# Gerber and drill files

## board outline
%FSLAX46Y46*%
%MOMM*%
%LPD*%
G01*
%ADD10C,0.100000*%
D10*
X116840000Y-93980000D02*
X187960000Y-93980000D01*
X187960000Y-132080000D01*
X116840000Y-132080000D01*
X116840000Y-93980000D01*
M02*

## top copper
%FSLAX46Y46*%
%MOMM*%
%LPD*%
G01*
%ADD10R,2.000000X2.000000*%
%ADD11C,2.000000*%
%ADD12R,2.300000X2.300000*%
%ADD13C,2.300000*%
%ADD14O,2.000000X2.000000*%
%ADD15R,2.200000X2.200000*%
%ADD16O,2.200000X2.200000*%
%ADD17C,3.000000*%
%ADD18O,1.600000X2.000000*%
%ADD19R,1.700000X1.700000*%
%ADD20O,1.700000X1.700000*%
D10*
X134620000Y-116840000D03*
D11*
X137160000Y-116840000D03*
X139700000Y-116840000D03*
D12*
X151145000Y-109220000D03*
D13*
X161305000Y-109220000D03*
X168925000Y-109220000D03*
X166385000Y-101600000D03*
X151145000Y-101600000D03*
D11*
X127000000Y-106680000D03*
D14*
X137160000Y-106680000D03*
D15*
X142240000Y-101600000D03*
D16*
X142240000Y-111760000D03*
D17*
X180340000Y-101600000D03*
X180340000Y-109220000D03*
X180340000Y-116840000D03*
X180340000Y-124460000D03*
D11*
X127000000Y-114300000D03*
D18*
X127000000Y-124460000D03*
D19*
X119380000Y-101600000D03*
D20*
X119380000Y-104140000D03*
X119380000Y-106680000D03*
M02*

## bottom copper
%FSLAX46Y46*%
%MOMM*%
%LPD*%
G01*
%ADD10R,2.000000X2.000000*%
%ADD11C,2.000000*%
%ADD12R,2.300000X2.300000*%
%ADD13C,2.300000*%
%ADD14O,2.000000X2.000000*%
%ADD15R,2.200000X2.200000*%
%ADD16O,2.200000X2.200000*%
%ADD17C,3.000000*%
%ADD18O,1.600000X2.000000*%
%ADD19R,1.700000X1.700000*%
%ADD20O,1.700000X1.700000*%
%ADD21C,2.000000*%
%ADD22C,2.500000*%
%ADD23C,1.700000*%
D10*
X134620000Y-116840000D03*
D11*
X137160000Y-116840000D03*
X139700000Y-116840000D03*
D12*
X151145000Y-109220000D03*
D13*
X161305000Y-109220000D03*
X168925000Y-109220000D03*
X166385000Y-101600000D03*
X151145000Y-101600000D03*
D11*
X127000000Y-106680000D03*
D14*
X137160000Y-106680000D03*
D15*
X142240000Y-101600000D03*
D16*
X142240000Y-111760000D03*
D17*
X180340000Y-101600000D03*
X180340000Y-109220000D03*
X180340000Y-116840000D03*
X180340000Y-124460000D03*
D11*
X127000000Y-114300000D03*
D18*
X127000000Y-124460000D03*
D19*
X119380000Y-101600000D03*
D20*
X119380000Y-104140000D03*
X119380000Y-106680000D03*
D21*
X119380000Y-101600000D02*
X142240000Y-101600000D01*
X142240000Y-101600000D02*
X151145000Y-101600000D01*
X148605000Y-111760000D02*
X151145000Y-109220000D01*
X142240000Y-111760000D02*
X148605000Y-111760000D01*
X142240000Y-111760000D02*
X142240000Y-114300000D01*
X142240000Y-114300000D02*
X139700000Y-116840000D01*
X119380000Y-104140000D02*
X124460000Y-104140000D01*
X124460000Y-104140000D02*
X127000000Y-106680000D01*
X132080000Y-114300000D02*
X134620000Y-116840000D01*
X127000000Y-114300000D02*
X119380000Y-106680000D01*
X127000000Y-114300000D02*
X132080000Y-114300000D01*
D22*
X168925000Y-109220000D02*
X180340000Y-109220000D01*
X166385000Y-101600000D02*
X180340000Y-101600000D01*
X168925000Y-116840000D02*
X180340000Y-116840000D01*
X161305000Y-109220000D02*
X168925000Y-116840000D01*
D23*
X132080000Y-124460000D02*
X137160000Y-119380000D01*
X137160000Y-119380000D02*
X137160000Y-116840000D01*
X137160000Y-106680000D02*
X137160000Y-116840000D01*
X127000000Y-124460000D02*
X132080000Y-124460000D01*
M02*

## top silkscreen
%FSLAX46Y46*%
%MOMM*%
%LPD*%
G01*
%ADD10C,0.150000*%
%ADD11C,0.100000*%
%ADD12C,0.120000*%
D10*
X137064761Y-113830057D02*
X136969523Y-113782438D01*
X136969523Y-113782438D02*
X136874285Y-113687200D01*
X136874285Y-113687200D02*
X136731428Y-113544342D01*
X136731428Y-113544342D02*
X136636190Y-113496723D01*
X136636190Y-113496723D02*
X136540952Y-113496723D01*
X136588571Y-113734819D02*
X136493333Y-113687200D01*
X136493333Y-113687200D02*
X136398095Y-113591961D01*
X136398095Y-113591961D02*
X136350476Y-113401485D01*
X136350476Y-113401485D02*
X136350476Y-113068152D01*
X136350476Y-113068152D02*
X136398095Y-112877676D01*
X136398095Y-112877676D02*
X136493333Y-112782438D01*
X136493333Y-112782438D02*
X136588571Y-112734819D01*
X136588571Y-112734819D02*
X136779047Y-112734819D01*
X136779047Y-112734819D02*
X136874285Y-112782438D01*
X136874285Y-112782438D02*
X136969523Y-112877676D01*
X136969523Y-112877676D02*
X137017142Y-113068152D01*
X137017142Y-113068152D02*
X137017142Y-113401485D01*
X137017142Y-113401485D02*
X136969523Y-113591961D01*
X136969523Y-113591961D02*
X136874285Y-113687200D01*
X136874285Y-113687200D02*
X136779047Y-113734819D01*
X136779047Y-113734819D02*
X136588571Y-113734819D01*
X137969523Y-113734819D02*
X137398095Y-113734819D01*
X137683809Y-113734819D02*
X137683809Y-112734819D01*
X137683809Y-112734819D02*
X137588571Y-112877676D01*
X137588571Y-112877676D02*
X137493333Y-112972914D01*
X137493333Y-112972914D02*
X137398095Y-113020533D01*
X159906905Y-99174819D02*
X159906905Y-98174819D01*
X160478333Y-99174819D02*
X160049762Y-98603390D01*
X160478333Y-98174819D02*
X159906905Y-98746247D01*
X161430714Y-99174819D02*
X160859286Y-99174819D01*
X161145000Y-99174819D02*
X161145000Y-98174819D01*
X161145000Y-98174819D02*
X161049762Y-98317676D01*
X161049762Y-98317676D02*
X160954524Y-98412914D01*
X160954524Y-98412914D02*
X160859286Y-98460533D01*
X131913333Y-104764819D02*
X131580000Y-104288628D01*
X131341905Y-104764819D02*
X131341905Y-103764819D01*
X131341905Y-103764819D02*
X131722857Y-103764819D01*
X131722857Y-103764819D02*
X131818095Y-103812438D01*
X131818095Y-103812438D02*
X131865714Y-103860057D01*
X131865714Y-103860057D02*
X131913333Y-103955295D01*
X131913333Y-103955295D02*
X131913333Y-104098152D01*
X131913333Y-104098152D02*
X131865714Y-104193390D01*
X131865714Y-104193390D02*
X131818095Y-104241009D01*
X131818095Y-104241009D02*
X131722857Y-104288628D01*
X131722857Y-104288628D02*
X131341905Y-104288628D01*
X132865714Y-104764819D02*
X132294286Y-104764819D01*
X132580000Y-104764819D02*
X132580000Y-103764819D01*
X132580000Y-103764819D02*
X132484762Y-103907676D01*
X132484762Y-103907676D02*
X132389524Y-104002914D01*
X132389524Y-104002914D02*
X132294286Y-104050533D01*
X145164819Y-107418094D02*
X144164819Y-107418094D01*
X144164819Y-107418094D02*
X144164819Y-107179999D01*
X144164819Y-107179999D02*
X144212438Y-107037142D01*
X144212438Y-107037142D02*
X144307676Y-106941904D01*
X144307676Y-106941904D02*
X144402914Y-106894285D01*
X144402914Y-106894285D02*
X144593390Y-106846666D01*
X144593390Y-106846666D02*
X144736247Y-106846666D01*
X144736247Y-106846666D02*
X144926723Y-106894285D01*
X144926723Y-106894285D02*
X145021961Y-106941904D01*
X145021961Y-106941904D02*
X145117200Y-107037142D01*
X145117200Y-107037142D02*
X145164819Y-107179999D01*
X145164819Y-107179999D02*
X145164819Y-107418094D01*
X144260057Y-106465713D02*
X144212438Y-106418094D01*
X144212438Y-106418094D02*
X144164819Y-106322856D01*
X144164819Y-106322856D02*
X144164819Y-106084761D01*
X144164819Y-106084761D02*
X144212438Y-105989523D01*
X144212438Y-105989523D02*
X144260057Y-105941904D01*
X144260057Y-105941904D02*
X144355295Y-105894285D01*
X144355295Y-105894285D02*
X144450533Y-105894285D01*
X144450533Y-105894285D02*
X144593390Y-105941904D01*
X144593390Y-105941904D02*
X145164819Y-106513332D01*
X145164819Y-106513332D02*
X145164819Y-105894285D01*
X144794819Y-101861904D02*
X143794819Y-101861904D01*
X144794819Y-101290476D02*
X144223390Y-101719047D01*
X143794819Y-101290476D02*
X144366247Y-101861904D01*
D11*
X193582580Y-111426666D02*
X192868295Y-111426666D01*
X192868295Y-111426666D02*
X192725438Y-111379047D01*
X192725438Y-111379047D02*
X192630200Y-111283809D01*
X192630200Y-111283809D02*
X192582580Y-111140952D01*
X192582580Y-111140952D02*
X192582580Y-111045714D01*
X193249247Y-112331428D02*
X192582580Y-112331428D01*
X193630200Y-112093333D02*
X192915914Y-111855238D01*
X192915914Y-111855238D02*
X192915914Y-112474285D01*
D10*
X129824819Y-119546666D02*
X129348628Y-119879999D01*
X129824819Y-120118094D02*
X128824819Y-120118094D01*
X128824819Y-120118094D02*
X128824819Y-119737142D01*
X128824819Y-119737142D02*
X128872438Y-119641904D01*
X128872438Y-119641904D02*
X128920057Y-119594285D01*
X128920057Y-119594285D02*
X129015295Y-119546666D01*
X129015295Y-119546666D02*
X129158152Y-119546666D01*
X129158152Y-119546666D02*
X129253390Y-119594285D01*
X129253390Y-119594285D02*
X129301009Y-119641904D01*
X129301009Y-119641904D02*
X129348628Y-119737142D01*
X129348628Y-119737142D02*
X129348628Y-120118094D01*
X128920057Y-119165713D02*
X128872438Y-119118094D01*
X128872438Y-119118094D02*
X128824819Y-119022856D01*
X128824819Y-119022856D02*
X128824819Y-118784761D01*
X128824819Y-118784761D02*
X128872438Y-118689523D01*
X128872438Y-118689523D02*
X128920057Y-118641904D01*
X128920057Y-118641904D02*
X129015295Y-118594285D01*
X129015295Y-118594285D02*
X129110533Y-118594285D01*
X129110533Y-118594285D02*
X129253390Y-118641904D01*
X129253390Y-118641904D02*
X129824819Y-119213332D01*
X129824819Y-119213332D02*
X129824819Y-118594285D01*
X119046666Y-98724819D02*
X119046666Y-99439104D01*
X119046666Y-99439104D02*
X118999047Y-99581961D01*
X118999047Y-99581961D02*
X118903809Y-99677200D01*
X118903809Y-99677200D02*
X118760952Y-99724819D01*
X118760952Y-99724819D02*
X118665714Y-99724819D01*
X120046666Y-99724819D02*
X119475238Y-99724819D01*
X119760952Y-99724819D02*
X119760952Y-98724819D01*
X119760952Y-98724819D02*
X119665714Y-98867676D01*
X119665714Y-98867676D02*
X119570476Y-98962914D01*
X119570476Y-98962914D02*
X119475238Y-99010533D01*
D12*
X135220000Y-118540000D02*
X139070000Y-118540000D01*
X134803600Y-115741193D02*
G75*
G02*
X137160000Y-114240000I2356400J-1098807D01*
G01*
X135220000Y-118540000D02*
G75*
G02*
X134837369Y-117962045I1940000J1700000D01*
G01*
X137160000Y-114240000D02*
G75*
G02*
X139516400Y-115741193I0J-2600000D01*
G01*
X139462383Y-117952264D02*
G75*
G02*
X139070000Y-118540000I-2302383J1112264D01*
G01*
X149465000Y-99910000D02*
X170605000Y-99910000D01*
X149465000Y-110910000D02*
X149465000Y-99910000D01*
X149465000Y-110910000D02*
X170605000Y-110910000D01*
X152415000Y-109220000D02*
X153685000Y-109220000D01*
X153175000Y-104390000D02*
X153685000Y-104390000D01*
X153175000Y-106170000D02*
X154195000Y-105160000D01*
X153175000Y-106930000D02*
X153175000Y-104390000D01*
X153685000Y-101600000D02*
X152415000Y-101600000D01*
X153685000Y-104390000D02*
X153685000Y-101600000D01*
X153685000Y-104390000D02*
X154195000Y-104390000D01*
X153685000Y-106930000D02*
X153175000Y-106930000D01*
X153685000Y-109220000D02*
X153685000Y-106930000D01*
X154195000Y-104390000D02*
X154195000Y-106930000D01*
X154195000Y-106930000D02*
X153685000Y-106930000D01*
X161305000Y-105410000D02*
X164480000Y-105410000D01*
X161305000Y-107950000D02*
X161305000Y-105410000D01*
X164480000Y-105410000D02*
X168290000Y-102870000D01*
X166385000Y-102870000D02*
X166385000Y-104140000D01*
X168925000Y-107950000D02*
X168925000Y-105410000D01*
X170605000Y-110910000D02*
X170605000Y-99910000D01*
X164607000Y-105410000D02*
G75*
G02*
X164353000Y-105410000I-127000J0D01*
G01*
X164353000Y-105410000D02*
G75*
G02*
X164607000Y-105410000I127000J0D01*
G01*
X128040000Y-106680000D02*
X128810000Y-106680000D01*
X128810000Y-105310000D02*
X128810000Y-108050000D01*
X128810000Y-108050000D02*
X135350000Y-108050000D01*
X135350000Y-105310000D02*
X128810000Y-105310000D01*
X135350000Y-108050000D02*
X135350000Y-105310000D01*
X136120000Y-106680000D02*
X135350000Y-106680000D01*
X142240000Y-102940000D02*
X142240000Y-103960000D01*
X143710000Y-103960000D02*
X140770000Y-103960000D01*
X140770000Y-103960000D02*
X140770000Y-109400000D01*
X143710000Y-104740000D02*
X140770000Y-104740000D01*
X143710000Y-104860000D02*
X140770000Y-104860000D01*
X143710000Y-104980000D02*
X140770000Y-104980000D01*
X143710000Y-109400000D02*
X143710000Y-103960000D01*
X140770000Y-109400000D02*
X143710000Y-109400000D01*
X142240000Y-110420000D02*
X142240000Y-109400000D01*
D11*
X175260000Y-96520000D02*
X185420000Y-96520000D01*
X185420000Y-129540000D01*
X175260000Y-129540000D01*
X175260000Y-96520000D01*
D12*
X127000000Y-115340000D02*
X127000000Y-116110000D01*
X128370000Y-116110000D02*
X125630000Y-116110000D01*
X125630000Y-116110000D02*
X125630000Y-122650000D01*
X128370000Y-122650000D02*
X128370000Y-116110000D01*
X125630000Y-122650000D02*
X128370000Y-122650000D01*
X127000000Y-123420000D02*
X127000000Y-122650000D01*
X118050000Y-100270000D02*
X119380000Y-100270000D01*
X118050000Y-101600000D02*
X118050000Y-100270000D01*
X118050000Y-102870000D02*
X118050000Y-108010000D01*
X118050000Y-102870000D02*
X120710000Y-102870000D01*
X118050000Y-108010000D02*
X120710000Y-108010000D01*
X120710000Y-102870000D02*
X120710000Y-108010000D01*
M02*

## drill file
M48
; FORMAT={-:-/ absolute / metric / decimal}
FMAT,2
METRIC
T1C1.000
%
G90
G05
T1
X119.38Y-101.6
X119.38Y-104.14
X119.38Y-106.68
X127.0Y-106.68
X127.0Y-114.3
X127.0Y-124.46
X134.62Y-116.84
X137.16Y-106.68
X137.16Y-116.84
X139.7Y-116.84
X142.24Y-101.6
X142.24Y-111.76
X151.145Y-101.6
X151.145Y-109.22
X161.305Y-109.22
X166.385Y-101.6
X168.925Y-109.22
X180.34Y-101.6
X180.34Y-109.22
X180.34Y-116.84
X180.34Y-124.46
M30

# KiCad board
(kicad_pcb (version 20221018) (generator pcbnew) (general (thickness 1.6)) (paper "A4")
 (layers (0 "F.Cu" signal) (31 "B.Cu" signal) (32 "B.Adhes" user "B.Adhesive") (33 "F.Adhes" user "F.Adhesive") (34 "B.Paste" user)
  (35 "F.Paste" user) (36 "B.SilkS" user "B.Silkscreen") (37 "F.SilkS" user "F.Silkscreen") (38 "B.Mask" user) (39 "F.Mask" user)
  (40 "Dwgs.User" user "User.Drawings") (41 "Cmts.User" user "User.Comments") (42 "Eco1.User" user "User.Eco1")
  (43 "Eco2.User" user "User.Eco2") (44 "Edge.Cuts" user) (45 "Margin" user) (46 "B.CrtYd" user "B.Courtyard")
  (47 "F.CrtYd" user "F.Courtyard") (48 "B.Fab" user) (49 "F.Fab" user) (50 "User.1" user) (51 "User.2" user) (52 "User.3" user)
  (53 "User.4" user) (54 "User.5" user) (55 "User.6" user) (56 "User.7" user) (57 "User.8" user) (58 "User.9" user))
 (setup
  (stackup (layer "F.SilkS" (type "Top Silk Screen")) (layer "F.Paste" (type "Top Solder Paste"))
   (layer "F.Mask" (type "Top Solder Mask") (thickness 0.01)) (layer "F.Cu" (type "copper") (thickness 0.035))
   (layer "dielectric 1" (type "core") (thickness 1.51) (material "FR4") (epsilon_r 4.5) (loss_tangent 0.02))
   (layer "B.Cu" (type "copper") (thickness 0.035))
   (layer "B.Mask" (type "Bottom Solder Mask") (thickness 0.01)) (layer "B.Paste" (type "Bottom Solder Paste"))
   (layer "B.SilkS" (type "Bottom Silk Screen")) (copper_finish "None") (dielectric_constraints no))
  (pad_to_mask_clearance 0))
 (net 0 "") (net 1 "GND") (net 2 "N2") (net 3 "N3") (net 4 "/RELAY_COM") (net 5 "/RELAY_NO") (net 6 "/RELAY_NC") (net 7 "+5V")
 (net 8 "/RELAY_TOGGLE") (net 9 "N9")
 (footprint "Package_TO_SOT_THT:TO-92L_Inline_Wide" (layer "F.Cu") (at 134.62 116.84)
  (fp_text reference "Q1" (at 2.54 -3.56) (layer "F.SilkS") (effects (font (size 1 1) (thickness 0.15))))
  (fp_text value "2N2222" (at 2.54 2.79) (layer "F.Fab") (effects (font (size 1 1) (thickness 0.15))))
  (fp_line (start 0.6 1.7) (end 4.45 1.7) (stroke (width 0.12) (type solid)) (layer "F.SilkS"))
  (fp_arc (start 0.1836 -1.098807) (mid 1.143021 -2.192817) (end 2.54 -2.6) (stroke (width 0.12) (type solid)) (layer "F.SilkS"))
  (fp_arc (start 0.6 1.7) (mid 0.389183 1.423933) (end 0.217369 1.122045) (stroke (width 0.12) (type solid)) (layer "F.SilkS"))
  (fp_arc (start 2.54 -2.6) (mid 3.936979 -2.192818) (end 4.8964 -1.098807) (stroke (width 0.12) (type solid)) (layer "F.SilkS"))
  (fp_arc (start 4.842383 1.112264) (mid 4.666594 1.419753) (end 4.45 1.7) (stroke (width 0.12) (type solid)) (layer "F.SilkS"))
  (pad "1" thru_hole rect (at 0 0) (size 2 2) (drill 1) (layers "*.Cu" "*.Mask") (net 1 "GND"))
  (pad "2" thru_hole circle (at 2.54 0) (size 2 2) (drill 1) (layers "*.Cu" "*.Mask") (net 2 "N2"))
  (pad "3" thru_hole circle (at 5.08 0) (size 2 2) (drill 1) (layers "*.Cu" "*.Mask") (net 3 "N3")))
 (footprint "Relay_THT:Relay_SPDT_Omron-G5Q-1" (layer "F.Cu") (at 151.145 109.22)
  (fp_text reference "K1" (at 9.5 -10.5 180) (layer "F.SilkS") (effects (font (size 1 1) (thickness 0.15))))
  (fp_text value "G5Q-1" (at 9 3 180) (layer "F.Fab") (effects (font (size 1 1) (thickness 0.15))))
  (fp_line (start -1.68 -9.31) (end 19.46 -9.31) (stroke (width 0.12) (type solid)) (layer "F.SilkS"))
  (fp_line (start -1.68 1.69) (end -1.68 -9.31) (stroke (width 0.12) (type solid)) (layer "F.SilkS"))
  (fp_line (start -1.68 1.69) (end 19.46 1.69) (stroke (width 0.12) (type solid)) (layer "F.SilkS"))
  (fp_line (start 1.27 0) (end 2.54 0) (stroke (width 0.12) (type solid)) (layer "F.SilkS"))
  (fp_line (start 2.03 -4.83) (end 2.54 -4.83) (stroke (width 0.12) (type solid)) (layer "F.SilkS"))
  (fp_line (start 2.03 -3.05) (end 3.05 -4.06) (stroke (width 0.12) (type solid)) (layer "F.SilkS"))
  (fp_line (start 2.03 -2.29) (end 2.03 -4.83) (stroke (width 0.12) (type solid)) (layer "F.SilkS"))
  (fp_line (start 2.54 -7.62) (end 1.27 -7.62) (stroke (width 0.12) (type solid)) (layer "F.SilkS"))
  (fp_line (start 2.54 -4.83) (end 2.54 -7.62) (stroke (width 0.12) (type solid)) (layer "F.SilkS"))
  (fp_line (start 2.54 -4.83) (end 3.05 -4.83) (stroke (width 0.12) (type solid)) (layer "F.SilkS"))
  (fp_line (start 2.54 -2.29) (end 2.03 -2.29) (stroke (width 0.12) (type solid)) (layer "F.SilkS"))
  (fp_line (start 2.54 0) (end 2.54 -2.29) (stroke (width 0.12) (type solid)) (layer "F.SilkS"))
  (fp_line (start 3.05 -4.83) (end 3.05 -2.29) (stroke (width 0.12) (type solid)) (layer "F.SilkS"))
  (fp_line (start 3.05 -2.29) (end 2.54 -2.29) (stroke (width 0.12) (type solid)) (layer "F.SilkS"))
  (fp_line (start 10.16 -3.81) (end 13.335 -3.81) (stroke (width 0.12) (type solid)) (layer "F.SilkS"))
  (fp_line (start 10.16 -1.27) (end 10.16 -3.81) (stroke (width 0.12) (type solid)) (layer "F.SilkS"))
  (fp_line (start 13.335 -3.81) (end 17.145 -6.35) (stroke (width 0.12) (type solid)) (layer "F.SilkS"))
  (fp_line (start 15.24 -6.35) (end 15.24 -5.08) (stroke (width 0.12) (type solid)) (layer "F.SilkS"))
  (fp_line (start 17.78 -1.27) (end 17.78 -3.81) (stroke (width 0.12) (type solid)) (layer "F.SilkS"))
  (fp_line (start 19.46 1.69) (end 19.46 -9.31) (stroke (width 0.12) (type solid)) (layer "F.SilkS"))
  (fp_circle (center 13.335 -3.81) (end 13.462 -3.81) (stroke (width 0.12) (type solid)) (fill none) (layer "F.SilkS"))
  (pad "1" thru_hole rect (at 0 0 180) (size 2.3 2.3) (drill 1) (layers "*.Cu" "*.Mask") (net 3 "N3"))
  (pad "2" thru_hole circle (at 10.16 0 180) (size 2.3 2.3) (drill 1) (layers "*.Cu" "*.Mask") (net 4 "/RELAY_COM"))
  (pad "3" thru_hole circle (at 17.78 0 180) (size 2.3 2.3) (drill 1) (layers "*.Cu" "*.Mask") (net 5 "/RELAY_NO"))
  (pad "4" thru_hole circle (at 15.24 -7.62 180) (size 2.3 2.3) (drill 1) (layers "*.Cu" "*.Mask") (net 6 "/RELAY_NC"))
  (pad "5" thru_hole circle (at 0 -7.62 180) (size 2.3 2.3) (drill 1) (layers "*.Cu" "*.Mask") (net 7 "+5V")))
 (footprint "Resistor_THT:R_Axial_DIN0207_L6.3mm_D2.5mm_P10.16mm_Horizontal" (layer "F.Cu") (at 127 106.68)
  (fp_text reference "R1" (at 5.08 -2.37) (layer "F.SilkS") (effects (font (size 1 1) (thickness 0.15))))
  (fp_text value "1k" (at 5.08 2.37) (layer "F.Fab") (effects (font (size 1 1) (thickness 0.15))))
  (fp_line (start 1.04 0) (end 1.81 0) (stroke (width 0.12) (type solid)) (layer "F.SilkS"))
  (fp_line (start 1.81 -1.37) (end 1.81 1.37) (stroke (width 0.12) (type solid)) (layer "F.SilkS"))
  (fp_line (start 1.81 1.37) (end 8.35 1.37) (stroke (width 0.12) (type solid)) (layer "F.SilkS"))
  (fp_line (start 8.35 -1.37) (end 1.81 -1.37) (stroke (width 0.12) (type solid)) (layer "F.SilkS"))
  (fp_line (start 8.35 1.37) (end 8.35 -1.37) (stroke (width 0.12) (type solid)) (layer "F.SilkS"))
  (fp_line (start 9.12 0) (end 8.35 0) (stroke (width 0.12) (type solid)) (layer "F.SilkS"))
  (pad "1" thru_hole circle (at 0 0) (size 2 2) (drill 1) (layers "*.Cu" "*.Mask") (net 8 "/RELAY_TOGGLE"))
  (pad "2" thru_hole oval (at 10.16 0) (size 2 2) (drill 1) (layers "*.Cu" "*.Mask") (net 2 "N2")))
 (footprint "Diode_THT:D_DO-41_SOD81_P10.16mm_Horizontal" (layer "F.Cu") (at 142.24 101.6 -90)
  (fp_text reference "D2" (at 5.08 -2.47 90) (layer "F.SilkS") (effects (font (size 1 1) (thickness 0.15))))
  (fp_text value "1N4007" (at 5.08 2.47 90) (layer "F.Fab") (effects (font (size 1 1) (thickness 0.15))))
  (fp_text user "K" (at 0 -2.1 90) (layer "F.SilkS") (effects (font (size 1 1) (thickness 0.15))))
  (fp_line (start 1.34 0) (end 2.36 0) (stroke (width 0.12) (type solid)) (layer "F.SilkS"))
  (fp_line (start 2.36 -1.47) (end 2.36 1.47) (stroke (width 0.12) (type solid)) (layer "F.SilkS"))
  (fp_line (start 2.36 1.47) (end 7.8 1.47) (stroke (width 0.12) (type solid)) (layer "F.SilkS"))
  (fp_line (start 3.14 -1.47) (end 3.14 1.47) (stroke (width 0.12) (type solid)) (layer "F.SilkS"))
  (fp_line (start 3.26 -1.47) (end 3.26 1.47) (stroke (width 0.12) (type solid)) (layer "F.SilkS"))
  (fp_line (start 3.38 -1.47) (end 3.38 1.47) (stroke (width 0.12) (type solid)) (layer "F.SilkS"))
  (fp_line (start 7.8 -1.47) (end 2.36 -1.47) (stroke (width 0.12) (type solid)) (layer "F.SilkS"))
  (fp_line (start 7.8 1.47) (end 7.8 -1.47) (stroke (width 0.12) (type solid)) (layer "F.SilkS"))
  (fp_line (start 8.82 0) (end 7.8 0) (stroke (width 0.12) (type solid)) (layer "F.SilkS"))
  (pad "1" thru_hole rect (at 0 0 270) (size 2.2 2.2) (drill 1) (layers "*.Cu" "*.Mask") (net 7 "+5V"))
  (pad "2" thru_hole oval (at 10.16 0 270) (size 2.2 2.2) (drill 1) (layers "*.Cu" "*.Mask") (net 3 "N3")))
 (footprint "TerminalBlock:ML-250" (layer "F.Cu") (at 190.5 111.76 -90)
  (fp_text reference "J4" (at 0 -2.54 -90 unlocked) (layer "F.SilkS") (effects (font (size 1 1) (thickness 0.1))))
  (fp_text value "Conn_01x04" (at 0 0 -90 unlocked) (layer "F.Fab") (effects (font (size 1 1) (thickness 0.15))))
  (fp_rect (start -15.24 5.08) (end 17.78 15.24) (stroke (width 0.1) (type default)) (fill none) (layer "F.SilkS"))
  (pad "1" thru_hole circle (at -10.16 10.16 270) (size 3 3) (drill 1) (layers "*.Cu" "*.Mask") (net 6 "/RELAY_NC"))
  (pad "2" thru_hole circle (at -2.54 10.16 270) (size 3 3) (drill 1) (layers "*.Cu" "*.Mask") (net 5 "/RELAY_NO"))
  (pad "3" thru_hole circle (at 5.08 10.16 270) (size 3 3) (drill 1) (layers "*.Cu" "*.Mask") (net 4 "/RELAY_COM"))
  (pad "4" thru_hole circle (at 12.7 10.16 270) (size 3 3) (drill 1) (layers "*.Cu" "*.Mask") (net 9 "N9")))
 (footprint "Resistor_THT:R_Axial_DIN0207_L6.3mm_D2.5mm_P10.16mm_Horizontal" (layer "F.Cu") (at 127 114.3 -90)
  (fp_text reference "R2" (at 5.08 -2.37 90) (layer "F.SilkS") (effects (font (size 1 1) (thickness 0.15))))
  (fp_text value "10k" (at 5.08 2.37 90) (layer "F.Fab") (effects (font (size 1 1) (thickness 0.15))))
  (fp_line (start 1.04 0) (end 1.81 0) (stroke (width 0.12) (type solid)) (layer "F.SilkS"))
  (fp_line (start 1.81 -1.37) (end 1.81 1.37) (stroke (width 0.12) (type solid)) (layer "F.SilkS"))
  (fp_line (start 1.81 1.37) (end 8.35 1.37) (stroke (width 0.12) (type solid)) (layer "F.SilkS"))
  (fp_line (start 8.35 -1.37) (end 1.81 -1.37) (stroke (width 0.12) (type solid)) (layer "F.SilkS"))
  (fp_line (start 8.35 1.37) (end 8.35 -1.37) (stroke (width 0.12) (type solid)) (layer "F.SilkS"))
  (fp_line (start 9.12 0) (end 8.35 0) (stroke (width 0.12) (type solid)) (layer "F.SilkS"))
  (pad "1" thru_hole circle (at 0 0 270) (size 2 2) (drill 1) (layers "*.Cu" "*.Mask") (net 1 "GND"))
  (pad "2" thru_hole oval (at 10.16 0 270) (size 2 1.6) (drill 1) (layers "*.Cu" "*.Mask") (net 2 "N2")))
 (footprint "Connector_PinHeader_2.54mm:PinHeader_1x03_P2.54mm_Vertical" (layer "F.Cu") (at 119.38 101.6)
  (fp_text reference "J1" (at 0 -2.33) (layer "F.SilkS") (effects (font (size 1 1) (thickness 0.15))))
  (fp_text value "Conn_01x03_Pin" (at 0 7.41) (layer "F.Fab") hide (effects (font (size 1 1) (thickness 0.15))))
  (fp_line (start -1.33 -1.33) (end 0 -1.33) (stroke (width 0.12) (type solid)) (layer "F.SilkS"))
  (fp_line (start -1.33 0) (end -1.33 -1.33) (stroke (width 0.12) (type solid)) (layer "F.SilkS"))
  (fp_line (start -1.33 1.27) (end -1.33 6.41) (stroke (width 0.12) (type solid)) (layer "F.SilkS"))
  (fp_line (start -1.33 1.27) (end 1.33 1.27) (stroke (width 0.12) (type solid)) (layer "F.SilkS"))
  (fp_line (start -1.33 6.41) (end 1.33 6.41) (stroke (width 0.12) (type solid)) (layer "F.SilkS"))
  (fp_line (start 1.33 1.27) (end 1.33 6.41) (stroke (width 0.12) (type solid)) (layer "F.SilkS"))
  (pad "1" thru_hole rect (at 0 0) (size 1.7 1.7) (drill 1) (layers "*.Cu" "*.Mask") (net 7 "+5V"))
  (pad "2" thru_hole oval (at 0 2.54) (size 1.7 1.7) (drill 1) (layers "*.Cu" "*.Mask") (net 8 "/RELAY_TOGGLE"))
  (pad "3" thru_hole oval (at 0 5.08) (size 1.7 1.7) (drill 1) (layers "*.Cu" "*.Mask") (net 1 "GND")))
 (gr_rect (start 116.84 93.98) (end 187.96 132.08) (stroke (width 0.1) (type default)) (fill none) (layer "Edge.Cuts"))
 (segment (start 119.38 101.6) (end 142.24 101.6) (width 2) (layer "B.Cu") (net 7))
 (segment (start 142.24 101.6) (end 151.145 101.6) (width 2) (layer "B.Cu") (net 7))
 (segment (start 148.605 111.76) (end 151.145 109.22) (width 2) (layer "B.Cu") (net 3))
 (segment (start 142.24 111.76) (end 148.605 111.76) (width 2) (layer "B.Cu") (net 3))
 (segment (start 142.24 111.76) (end 142.24 114.3) (width 2) (layer "B.Cu") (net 3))
 (segment (start 142.24 114.3) (end 139.7 116.84) (width 2) (layer "B.Cu") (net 3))
 (segment (start 119.38 104.14) (end 124.46 104.14) (width 2) (layer "B.Cu") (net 8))
 (segment (start 124.46 104.14) (end 127 106.68) (width 2) (layer "B.Cu") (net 8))
 (segment (start 132.08 114.3) (end 134.62 116.84) (width 2) (layer "B.Cu") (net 1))
 (segment (start 127 114.3) (end 119.38 106.68) (width 2) (layer "B.Cu") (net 1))
 (segment (start 127 114.3) (end 132.08 114.3) (width 2) (layer "B.Cu") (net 1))
 (segment (start 168.925 109.22) (end 180.34 109.22) (width 2.5) (layer "B.Cu") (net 5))
 (segment (start 166.385 101.6) (end 180.34 101.6) (width 2.5) (layer "B.Cu") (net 6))
 (segment (start 168.925 116.84) (end 180.34 116.84) (width 2.5) (layer "B.Cu") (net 4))
 (segment (start 161.305 109.22) (end 168.925 116.84) (width 2.5) (layer "B.Cu") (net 4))
 (segment (start 132.08 124.46) (end 137.16 119.38) (width 1.7) (layer "B.Cu") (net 2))
 (segment (start 137.16 119.38) (end 137.16 116.84) (width 1.7) (layer "B.Cu") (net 2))
 (segment (start 137.16 106.68) (end 137.16 116.84) (width 1.7) (layer "B.Cu") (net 2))
 (segment (start 127 124.46) (end 132.08 124.46) (width 1.7) (layer "B.Cu") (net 2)))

